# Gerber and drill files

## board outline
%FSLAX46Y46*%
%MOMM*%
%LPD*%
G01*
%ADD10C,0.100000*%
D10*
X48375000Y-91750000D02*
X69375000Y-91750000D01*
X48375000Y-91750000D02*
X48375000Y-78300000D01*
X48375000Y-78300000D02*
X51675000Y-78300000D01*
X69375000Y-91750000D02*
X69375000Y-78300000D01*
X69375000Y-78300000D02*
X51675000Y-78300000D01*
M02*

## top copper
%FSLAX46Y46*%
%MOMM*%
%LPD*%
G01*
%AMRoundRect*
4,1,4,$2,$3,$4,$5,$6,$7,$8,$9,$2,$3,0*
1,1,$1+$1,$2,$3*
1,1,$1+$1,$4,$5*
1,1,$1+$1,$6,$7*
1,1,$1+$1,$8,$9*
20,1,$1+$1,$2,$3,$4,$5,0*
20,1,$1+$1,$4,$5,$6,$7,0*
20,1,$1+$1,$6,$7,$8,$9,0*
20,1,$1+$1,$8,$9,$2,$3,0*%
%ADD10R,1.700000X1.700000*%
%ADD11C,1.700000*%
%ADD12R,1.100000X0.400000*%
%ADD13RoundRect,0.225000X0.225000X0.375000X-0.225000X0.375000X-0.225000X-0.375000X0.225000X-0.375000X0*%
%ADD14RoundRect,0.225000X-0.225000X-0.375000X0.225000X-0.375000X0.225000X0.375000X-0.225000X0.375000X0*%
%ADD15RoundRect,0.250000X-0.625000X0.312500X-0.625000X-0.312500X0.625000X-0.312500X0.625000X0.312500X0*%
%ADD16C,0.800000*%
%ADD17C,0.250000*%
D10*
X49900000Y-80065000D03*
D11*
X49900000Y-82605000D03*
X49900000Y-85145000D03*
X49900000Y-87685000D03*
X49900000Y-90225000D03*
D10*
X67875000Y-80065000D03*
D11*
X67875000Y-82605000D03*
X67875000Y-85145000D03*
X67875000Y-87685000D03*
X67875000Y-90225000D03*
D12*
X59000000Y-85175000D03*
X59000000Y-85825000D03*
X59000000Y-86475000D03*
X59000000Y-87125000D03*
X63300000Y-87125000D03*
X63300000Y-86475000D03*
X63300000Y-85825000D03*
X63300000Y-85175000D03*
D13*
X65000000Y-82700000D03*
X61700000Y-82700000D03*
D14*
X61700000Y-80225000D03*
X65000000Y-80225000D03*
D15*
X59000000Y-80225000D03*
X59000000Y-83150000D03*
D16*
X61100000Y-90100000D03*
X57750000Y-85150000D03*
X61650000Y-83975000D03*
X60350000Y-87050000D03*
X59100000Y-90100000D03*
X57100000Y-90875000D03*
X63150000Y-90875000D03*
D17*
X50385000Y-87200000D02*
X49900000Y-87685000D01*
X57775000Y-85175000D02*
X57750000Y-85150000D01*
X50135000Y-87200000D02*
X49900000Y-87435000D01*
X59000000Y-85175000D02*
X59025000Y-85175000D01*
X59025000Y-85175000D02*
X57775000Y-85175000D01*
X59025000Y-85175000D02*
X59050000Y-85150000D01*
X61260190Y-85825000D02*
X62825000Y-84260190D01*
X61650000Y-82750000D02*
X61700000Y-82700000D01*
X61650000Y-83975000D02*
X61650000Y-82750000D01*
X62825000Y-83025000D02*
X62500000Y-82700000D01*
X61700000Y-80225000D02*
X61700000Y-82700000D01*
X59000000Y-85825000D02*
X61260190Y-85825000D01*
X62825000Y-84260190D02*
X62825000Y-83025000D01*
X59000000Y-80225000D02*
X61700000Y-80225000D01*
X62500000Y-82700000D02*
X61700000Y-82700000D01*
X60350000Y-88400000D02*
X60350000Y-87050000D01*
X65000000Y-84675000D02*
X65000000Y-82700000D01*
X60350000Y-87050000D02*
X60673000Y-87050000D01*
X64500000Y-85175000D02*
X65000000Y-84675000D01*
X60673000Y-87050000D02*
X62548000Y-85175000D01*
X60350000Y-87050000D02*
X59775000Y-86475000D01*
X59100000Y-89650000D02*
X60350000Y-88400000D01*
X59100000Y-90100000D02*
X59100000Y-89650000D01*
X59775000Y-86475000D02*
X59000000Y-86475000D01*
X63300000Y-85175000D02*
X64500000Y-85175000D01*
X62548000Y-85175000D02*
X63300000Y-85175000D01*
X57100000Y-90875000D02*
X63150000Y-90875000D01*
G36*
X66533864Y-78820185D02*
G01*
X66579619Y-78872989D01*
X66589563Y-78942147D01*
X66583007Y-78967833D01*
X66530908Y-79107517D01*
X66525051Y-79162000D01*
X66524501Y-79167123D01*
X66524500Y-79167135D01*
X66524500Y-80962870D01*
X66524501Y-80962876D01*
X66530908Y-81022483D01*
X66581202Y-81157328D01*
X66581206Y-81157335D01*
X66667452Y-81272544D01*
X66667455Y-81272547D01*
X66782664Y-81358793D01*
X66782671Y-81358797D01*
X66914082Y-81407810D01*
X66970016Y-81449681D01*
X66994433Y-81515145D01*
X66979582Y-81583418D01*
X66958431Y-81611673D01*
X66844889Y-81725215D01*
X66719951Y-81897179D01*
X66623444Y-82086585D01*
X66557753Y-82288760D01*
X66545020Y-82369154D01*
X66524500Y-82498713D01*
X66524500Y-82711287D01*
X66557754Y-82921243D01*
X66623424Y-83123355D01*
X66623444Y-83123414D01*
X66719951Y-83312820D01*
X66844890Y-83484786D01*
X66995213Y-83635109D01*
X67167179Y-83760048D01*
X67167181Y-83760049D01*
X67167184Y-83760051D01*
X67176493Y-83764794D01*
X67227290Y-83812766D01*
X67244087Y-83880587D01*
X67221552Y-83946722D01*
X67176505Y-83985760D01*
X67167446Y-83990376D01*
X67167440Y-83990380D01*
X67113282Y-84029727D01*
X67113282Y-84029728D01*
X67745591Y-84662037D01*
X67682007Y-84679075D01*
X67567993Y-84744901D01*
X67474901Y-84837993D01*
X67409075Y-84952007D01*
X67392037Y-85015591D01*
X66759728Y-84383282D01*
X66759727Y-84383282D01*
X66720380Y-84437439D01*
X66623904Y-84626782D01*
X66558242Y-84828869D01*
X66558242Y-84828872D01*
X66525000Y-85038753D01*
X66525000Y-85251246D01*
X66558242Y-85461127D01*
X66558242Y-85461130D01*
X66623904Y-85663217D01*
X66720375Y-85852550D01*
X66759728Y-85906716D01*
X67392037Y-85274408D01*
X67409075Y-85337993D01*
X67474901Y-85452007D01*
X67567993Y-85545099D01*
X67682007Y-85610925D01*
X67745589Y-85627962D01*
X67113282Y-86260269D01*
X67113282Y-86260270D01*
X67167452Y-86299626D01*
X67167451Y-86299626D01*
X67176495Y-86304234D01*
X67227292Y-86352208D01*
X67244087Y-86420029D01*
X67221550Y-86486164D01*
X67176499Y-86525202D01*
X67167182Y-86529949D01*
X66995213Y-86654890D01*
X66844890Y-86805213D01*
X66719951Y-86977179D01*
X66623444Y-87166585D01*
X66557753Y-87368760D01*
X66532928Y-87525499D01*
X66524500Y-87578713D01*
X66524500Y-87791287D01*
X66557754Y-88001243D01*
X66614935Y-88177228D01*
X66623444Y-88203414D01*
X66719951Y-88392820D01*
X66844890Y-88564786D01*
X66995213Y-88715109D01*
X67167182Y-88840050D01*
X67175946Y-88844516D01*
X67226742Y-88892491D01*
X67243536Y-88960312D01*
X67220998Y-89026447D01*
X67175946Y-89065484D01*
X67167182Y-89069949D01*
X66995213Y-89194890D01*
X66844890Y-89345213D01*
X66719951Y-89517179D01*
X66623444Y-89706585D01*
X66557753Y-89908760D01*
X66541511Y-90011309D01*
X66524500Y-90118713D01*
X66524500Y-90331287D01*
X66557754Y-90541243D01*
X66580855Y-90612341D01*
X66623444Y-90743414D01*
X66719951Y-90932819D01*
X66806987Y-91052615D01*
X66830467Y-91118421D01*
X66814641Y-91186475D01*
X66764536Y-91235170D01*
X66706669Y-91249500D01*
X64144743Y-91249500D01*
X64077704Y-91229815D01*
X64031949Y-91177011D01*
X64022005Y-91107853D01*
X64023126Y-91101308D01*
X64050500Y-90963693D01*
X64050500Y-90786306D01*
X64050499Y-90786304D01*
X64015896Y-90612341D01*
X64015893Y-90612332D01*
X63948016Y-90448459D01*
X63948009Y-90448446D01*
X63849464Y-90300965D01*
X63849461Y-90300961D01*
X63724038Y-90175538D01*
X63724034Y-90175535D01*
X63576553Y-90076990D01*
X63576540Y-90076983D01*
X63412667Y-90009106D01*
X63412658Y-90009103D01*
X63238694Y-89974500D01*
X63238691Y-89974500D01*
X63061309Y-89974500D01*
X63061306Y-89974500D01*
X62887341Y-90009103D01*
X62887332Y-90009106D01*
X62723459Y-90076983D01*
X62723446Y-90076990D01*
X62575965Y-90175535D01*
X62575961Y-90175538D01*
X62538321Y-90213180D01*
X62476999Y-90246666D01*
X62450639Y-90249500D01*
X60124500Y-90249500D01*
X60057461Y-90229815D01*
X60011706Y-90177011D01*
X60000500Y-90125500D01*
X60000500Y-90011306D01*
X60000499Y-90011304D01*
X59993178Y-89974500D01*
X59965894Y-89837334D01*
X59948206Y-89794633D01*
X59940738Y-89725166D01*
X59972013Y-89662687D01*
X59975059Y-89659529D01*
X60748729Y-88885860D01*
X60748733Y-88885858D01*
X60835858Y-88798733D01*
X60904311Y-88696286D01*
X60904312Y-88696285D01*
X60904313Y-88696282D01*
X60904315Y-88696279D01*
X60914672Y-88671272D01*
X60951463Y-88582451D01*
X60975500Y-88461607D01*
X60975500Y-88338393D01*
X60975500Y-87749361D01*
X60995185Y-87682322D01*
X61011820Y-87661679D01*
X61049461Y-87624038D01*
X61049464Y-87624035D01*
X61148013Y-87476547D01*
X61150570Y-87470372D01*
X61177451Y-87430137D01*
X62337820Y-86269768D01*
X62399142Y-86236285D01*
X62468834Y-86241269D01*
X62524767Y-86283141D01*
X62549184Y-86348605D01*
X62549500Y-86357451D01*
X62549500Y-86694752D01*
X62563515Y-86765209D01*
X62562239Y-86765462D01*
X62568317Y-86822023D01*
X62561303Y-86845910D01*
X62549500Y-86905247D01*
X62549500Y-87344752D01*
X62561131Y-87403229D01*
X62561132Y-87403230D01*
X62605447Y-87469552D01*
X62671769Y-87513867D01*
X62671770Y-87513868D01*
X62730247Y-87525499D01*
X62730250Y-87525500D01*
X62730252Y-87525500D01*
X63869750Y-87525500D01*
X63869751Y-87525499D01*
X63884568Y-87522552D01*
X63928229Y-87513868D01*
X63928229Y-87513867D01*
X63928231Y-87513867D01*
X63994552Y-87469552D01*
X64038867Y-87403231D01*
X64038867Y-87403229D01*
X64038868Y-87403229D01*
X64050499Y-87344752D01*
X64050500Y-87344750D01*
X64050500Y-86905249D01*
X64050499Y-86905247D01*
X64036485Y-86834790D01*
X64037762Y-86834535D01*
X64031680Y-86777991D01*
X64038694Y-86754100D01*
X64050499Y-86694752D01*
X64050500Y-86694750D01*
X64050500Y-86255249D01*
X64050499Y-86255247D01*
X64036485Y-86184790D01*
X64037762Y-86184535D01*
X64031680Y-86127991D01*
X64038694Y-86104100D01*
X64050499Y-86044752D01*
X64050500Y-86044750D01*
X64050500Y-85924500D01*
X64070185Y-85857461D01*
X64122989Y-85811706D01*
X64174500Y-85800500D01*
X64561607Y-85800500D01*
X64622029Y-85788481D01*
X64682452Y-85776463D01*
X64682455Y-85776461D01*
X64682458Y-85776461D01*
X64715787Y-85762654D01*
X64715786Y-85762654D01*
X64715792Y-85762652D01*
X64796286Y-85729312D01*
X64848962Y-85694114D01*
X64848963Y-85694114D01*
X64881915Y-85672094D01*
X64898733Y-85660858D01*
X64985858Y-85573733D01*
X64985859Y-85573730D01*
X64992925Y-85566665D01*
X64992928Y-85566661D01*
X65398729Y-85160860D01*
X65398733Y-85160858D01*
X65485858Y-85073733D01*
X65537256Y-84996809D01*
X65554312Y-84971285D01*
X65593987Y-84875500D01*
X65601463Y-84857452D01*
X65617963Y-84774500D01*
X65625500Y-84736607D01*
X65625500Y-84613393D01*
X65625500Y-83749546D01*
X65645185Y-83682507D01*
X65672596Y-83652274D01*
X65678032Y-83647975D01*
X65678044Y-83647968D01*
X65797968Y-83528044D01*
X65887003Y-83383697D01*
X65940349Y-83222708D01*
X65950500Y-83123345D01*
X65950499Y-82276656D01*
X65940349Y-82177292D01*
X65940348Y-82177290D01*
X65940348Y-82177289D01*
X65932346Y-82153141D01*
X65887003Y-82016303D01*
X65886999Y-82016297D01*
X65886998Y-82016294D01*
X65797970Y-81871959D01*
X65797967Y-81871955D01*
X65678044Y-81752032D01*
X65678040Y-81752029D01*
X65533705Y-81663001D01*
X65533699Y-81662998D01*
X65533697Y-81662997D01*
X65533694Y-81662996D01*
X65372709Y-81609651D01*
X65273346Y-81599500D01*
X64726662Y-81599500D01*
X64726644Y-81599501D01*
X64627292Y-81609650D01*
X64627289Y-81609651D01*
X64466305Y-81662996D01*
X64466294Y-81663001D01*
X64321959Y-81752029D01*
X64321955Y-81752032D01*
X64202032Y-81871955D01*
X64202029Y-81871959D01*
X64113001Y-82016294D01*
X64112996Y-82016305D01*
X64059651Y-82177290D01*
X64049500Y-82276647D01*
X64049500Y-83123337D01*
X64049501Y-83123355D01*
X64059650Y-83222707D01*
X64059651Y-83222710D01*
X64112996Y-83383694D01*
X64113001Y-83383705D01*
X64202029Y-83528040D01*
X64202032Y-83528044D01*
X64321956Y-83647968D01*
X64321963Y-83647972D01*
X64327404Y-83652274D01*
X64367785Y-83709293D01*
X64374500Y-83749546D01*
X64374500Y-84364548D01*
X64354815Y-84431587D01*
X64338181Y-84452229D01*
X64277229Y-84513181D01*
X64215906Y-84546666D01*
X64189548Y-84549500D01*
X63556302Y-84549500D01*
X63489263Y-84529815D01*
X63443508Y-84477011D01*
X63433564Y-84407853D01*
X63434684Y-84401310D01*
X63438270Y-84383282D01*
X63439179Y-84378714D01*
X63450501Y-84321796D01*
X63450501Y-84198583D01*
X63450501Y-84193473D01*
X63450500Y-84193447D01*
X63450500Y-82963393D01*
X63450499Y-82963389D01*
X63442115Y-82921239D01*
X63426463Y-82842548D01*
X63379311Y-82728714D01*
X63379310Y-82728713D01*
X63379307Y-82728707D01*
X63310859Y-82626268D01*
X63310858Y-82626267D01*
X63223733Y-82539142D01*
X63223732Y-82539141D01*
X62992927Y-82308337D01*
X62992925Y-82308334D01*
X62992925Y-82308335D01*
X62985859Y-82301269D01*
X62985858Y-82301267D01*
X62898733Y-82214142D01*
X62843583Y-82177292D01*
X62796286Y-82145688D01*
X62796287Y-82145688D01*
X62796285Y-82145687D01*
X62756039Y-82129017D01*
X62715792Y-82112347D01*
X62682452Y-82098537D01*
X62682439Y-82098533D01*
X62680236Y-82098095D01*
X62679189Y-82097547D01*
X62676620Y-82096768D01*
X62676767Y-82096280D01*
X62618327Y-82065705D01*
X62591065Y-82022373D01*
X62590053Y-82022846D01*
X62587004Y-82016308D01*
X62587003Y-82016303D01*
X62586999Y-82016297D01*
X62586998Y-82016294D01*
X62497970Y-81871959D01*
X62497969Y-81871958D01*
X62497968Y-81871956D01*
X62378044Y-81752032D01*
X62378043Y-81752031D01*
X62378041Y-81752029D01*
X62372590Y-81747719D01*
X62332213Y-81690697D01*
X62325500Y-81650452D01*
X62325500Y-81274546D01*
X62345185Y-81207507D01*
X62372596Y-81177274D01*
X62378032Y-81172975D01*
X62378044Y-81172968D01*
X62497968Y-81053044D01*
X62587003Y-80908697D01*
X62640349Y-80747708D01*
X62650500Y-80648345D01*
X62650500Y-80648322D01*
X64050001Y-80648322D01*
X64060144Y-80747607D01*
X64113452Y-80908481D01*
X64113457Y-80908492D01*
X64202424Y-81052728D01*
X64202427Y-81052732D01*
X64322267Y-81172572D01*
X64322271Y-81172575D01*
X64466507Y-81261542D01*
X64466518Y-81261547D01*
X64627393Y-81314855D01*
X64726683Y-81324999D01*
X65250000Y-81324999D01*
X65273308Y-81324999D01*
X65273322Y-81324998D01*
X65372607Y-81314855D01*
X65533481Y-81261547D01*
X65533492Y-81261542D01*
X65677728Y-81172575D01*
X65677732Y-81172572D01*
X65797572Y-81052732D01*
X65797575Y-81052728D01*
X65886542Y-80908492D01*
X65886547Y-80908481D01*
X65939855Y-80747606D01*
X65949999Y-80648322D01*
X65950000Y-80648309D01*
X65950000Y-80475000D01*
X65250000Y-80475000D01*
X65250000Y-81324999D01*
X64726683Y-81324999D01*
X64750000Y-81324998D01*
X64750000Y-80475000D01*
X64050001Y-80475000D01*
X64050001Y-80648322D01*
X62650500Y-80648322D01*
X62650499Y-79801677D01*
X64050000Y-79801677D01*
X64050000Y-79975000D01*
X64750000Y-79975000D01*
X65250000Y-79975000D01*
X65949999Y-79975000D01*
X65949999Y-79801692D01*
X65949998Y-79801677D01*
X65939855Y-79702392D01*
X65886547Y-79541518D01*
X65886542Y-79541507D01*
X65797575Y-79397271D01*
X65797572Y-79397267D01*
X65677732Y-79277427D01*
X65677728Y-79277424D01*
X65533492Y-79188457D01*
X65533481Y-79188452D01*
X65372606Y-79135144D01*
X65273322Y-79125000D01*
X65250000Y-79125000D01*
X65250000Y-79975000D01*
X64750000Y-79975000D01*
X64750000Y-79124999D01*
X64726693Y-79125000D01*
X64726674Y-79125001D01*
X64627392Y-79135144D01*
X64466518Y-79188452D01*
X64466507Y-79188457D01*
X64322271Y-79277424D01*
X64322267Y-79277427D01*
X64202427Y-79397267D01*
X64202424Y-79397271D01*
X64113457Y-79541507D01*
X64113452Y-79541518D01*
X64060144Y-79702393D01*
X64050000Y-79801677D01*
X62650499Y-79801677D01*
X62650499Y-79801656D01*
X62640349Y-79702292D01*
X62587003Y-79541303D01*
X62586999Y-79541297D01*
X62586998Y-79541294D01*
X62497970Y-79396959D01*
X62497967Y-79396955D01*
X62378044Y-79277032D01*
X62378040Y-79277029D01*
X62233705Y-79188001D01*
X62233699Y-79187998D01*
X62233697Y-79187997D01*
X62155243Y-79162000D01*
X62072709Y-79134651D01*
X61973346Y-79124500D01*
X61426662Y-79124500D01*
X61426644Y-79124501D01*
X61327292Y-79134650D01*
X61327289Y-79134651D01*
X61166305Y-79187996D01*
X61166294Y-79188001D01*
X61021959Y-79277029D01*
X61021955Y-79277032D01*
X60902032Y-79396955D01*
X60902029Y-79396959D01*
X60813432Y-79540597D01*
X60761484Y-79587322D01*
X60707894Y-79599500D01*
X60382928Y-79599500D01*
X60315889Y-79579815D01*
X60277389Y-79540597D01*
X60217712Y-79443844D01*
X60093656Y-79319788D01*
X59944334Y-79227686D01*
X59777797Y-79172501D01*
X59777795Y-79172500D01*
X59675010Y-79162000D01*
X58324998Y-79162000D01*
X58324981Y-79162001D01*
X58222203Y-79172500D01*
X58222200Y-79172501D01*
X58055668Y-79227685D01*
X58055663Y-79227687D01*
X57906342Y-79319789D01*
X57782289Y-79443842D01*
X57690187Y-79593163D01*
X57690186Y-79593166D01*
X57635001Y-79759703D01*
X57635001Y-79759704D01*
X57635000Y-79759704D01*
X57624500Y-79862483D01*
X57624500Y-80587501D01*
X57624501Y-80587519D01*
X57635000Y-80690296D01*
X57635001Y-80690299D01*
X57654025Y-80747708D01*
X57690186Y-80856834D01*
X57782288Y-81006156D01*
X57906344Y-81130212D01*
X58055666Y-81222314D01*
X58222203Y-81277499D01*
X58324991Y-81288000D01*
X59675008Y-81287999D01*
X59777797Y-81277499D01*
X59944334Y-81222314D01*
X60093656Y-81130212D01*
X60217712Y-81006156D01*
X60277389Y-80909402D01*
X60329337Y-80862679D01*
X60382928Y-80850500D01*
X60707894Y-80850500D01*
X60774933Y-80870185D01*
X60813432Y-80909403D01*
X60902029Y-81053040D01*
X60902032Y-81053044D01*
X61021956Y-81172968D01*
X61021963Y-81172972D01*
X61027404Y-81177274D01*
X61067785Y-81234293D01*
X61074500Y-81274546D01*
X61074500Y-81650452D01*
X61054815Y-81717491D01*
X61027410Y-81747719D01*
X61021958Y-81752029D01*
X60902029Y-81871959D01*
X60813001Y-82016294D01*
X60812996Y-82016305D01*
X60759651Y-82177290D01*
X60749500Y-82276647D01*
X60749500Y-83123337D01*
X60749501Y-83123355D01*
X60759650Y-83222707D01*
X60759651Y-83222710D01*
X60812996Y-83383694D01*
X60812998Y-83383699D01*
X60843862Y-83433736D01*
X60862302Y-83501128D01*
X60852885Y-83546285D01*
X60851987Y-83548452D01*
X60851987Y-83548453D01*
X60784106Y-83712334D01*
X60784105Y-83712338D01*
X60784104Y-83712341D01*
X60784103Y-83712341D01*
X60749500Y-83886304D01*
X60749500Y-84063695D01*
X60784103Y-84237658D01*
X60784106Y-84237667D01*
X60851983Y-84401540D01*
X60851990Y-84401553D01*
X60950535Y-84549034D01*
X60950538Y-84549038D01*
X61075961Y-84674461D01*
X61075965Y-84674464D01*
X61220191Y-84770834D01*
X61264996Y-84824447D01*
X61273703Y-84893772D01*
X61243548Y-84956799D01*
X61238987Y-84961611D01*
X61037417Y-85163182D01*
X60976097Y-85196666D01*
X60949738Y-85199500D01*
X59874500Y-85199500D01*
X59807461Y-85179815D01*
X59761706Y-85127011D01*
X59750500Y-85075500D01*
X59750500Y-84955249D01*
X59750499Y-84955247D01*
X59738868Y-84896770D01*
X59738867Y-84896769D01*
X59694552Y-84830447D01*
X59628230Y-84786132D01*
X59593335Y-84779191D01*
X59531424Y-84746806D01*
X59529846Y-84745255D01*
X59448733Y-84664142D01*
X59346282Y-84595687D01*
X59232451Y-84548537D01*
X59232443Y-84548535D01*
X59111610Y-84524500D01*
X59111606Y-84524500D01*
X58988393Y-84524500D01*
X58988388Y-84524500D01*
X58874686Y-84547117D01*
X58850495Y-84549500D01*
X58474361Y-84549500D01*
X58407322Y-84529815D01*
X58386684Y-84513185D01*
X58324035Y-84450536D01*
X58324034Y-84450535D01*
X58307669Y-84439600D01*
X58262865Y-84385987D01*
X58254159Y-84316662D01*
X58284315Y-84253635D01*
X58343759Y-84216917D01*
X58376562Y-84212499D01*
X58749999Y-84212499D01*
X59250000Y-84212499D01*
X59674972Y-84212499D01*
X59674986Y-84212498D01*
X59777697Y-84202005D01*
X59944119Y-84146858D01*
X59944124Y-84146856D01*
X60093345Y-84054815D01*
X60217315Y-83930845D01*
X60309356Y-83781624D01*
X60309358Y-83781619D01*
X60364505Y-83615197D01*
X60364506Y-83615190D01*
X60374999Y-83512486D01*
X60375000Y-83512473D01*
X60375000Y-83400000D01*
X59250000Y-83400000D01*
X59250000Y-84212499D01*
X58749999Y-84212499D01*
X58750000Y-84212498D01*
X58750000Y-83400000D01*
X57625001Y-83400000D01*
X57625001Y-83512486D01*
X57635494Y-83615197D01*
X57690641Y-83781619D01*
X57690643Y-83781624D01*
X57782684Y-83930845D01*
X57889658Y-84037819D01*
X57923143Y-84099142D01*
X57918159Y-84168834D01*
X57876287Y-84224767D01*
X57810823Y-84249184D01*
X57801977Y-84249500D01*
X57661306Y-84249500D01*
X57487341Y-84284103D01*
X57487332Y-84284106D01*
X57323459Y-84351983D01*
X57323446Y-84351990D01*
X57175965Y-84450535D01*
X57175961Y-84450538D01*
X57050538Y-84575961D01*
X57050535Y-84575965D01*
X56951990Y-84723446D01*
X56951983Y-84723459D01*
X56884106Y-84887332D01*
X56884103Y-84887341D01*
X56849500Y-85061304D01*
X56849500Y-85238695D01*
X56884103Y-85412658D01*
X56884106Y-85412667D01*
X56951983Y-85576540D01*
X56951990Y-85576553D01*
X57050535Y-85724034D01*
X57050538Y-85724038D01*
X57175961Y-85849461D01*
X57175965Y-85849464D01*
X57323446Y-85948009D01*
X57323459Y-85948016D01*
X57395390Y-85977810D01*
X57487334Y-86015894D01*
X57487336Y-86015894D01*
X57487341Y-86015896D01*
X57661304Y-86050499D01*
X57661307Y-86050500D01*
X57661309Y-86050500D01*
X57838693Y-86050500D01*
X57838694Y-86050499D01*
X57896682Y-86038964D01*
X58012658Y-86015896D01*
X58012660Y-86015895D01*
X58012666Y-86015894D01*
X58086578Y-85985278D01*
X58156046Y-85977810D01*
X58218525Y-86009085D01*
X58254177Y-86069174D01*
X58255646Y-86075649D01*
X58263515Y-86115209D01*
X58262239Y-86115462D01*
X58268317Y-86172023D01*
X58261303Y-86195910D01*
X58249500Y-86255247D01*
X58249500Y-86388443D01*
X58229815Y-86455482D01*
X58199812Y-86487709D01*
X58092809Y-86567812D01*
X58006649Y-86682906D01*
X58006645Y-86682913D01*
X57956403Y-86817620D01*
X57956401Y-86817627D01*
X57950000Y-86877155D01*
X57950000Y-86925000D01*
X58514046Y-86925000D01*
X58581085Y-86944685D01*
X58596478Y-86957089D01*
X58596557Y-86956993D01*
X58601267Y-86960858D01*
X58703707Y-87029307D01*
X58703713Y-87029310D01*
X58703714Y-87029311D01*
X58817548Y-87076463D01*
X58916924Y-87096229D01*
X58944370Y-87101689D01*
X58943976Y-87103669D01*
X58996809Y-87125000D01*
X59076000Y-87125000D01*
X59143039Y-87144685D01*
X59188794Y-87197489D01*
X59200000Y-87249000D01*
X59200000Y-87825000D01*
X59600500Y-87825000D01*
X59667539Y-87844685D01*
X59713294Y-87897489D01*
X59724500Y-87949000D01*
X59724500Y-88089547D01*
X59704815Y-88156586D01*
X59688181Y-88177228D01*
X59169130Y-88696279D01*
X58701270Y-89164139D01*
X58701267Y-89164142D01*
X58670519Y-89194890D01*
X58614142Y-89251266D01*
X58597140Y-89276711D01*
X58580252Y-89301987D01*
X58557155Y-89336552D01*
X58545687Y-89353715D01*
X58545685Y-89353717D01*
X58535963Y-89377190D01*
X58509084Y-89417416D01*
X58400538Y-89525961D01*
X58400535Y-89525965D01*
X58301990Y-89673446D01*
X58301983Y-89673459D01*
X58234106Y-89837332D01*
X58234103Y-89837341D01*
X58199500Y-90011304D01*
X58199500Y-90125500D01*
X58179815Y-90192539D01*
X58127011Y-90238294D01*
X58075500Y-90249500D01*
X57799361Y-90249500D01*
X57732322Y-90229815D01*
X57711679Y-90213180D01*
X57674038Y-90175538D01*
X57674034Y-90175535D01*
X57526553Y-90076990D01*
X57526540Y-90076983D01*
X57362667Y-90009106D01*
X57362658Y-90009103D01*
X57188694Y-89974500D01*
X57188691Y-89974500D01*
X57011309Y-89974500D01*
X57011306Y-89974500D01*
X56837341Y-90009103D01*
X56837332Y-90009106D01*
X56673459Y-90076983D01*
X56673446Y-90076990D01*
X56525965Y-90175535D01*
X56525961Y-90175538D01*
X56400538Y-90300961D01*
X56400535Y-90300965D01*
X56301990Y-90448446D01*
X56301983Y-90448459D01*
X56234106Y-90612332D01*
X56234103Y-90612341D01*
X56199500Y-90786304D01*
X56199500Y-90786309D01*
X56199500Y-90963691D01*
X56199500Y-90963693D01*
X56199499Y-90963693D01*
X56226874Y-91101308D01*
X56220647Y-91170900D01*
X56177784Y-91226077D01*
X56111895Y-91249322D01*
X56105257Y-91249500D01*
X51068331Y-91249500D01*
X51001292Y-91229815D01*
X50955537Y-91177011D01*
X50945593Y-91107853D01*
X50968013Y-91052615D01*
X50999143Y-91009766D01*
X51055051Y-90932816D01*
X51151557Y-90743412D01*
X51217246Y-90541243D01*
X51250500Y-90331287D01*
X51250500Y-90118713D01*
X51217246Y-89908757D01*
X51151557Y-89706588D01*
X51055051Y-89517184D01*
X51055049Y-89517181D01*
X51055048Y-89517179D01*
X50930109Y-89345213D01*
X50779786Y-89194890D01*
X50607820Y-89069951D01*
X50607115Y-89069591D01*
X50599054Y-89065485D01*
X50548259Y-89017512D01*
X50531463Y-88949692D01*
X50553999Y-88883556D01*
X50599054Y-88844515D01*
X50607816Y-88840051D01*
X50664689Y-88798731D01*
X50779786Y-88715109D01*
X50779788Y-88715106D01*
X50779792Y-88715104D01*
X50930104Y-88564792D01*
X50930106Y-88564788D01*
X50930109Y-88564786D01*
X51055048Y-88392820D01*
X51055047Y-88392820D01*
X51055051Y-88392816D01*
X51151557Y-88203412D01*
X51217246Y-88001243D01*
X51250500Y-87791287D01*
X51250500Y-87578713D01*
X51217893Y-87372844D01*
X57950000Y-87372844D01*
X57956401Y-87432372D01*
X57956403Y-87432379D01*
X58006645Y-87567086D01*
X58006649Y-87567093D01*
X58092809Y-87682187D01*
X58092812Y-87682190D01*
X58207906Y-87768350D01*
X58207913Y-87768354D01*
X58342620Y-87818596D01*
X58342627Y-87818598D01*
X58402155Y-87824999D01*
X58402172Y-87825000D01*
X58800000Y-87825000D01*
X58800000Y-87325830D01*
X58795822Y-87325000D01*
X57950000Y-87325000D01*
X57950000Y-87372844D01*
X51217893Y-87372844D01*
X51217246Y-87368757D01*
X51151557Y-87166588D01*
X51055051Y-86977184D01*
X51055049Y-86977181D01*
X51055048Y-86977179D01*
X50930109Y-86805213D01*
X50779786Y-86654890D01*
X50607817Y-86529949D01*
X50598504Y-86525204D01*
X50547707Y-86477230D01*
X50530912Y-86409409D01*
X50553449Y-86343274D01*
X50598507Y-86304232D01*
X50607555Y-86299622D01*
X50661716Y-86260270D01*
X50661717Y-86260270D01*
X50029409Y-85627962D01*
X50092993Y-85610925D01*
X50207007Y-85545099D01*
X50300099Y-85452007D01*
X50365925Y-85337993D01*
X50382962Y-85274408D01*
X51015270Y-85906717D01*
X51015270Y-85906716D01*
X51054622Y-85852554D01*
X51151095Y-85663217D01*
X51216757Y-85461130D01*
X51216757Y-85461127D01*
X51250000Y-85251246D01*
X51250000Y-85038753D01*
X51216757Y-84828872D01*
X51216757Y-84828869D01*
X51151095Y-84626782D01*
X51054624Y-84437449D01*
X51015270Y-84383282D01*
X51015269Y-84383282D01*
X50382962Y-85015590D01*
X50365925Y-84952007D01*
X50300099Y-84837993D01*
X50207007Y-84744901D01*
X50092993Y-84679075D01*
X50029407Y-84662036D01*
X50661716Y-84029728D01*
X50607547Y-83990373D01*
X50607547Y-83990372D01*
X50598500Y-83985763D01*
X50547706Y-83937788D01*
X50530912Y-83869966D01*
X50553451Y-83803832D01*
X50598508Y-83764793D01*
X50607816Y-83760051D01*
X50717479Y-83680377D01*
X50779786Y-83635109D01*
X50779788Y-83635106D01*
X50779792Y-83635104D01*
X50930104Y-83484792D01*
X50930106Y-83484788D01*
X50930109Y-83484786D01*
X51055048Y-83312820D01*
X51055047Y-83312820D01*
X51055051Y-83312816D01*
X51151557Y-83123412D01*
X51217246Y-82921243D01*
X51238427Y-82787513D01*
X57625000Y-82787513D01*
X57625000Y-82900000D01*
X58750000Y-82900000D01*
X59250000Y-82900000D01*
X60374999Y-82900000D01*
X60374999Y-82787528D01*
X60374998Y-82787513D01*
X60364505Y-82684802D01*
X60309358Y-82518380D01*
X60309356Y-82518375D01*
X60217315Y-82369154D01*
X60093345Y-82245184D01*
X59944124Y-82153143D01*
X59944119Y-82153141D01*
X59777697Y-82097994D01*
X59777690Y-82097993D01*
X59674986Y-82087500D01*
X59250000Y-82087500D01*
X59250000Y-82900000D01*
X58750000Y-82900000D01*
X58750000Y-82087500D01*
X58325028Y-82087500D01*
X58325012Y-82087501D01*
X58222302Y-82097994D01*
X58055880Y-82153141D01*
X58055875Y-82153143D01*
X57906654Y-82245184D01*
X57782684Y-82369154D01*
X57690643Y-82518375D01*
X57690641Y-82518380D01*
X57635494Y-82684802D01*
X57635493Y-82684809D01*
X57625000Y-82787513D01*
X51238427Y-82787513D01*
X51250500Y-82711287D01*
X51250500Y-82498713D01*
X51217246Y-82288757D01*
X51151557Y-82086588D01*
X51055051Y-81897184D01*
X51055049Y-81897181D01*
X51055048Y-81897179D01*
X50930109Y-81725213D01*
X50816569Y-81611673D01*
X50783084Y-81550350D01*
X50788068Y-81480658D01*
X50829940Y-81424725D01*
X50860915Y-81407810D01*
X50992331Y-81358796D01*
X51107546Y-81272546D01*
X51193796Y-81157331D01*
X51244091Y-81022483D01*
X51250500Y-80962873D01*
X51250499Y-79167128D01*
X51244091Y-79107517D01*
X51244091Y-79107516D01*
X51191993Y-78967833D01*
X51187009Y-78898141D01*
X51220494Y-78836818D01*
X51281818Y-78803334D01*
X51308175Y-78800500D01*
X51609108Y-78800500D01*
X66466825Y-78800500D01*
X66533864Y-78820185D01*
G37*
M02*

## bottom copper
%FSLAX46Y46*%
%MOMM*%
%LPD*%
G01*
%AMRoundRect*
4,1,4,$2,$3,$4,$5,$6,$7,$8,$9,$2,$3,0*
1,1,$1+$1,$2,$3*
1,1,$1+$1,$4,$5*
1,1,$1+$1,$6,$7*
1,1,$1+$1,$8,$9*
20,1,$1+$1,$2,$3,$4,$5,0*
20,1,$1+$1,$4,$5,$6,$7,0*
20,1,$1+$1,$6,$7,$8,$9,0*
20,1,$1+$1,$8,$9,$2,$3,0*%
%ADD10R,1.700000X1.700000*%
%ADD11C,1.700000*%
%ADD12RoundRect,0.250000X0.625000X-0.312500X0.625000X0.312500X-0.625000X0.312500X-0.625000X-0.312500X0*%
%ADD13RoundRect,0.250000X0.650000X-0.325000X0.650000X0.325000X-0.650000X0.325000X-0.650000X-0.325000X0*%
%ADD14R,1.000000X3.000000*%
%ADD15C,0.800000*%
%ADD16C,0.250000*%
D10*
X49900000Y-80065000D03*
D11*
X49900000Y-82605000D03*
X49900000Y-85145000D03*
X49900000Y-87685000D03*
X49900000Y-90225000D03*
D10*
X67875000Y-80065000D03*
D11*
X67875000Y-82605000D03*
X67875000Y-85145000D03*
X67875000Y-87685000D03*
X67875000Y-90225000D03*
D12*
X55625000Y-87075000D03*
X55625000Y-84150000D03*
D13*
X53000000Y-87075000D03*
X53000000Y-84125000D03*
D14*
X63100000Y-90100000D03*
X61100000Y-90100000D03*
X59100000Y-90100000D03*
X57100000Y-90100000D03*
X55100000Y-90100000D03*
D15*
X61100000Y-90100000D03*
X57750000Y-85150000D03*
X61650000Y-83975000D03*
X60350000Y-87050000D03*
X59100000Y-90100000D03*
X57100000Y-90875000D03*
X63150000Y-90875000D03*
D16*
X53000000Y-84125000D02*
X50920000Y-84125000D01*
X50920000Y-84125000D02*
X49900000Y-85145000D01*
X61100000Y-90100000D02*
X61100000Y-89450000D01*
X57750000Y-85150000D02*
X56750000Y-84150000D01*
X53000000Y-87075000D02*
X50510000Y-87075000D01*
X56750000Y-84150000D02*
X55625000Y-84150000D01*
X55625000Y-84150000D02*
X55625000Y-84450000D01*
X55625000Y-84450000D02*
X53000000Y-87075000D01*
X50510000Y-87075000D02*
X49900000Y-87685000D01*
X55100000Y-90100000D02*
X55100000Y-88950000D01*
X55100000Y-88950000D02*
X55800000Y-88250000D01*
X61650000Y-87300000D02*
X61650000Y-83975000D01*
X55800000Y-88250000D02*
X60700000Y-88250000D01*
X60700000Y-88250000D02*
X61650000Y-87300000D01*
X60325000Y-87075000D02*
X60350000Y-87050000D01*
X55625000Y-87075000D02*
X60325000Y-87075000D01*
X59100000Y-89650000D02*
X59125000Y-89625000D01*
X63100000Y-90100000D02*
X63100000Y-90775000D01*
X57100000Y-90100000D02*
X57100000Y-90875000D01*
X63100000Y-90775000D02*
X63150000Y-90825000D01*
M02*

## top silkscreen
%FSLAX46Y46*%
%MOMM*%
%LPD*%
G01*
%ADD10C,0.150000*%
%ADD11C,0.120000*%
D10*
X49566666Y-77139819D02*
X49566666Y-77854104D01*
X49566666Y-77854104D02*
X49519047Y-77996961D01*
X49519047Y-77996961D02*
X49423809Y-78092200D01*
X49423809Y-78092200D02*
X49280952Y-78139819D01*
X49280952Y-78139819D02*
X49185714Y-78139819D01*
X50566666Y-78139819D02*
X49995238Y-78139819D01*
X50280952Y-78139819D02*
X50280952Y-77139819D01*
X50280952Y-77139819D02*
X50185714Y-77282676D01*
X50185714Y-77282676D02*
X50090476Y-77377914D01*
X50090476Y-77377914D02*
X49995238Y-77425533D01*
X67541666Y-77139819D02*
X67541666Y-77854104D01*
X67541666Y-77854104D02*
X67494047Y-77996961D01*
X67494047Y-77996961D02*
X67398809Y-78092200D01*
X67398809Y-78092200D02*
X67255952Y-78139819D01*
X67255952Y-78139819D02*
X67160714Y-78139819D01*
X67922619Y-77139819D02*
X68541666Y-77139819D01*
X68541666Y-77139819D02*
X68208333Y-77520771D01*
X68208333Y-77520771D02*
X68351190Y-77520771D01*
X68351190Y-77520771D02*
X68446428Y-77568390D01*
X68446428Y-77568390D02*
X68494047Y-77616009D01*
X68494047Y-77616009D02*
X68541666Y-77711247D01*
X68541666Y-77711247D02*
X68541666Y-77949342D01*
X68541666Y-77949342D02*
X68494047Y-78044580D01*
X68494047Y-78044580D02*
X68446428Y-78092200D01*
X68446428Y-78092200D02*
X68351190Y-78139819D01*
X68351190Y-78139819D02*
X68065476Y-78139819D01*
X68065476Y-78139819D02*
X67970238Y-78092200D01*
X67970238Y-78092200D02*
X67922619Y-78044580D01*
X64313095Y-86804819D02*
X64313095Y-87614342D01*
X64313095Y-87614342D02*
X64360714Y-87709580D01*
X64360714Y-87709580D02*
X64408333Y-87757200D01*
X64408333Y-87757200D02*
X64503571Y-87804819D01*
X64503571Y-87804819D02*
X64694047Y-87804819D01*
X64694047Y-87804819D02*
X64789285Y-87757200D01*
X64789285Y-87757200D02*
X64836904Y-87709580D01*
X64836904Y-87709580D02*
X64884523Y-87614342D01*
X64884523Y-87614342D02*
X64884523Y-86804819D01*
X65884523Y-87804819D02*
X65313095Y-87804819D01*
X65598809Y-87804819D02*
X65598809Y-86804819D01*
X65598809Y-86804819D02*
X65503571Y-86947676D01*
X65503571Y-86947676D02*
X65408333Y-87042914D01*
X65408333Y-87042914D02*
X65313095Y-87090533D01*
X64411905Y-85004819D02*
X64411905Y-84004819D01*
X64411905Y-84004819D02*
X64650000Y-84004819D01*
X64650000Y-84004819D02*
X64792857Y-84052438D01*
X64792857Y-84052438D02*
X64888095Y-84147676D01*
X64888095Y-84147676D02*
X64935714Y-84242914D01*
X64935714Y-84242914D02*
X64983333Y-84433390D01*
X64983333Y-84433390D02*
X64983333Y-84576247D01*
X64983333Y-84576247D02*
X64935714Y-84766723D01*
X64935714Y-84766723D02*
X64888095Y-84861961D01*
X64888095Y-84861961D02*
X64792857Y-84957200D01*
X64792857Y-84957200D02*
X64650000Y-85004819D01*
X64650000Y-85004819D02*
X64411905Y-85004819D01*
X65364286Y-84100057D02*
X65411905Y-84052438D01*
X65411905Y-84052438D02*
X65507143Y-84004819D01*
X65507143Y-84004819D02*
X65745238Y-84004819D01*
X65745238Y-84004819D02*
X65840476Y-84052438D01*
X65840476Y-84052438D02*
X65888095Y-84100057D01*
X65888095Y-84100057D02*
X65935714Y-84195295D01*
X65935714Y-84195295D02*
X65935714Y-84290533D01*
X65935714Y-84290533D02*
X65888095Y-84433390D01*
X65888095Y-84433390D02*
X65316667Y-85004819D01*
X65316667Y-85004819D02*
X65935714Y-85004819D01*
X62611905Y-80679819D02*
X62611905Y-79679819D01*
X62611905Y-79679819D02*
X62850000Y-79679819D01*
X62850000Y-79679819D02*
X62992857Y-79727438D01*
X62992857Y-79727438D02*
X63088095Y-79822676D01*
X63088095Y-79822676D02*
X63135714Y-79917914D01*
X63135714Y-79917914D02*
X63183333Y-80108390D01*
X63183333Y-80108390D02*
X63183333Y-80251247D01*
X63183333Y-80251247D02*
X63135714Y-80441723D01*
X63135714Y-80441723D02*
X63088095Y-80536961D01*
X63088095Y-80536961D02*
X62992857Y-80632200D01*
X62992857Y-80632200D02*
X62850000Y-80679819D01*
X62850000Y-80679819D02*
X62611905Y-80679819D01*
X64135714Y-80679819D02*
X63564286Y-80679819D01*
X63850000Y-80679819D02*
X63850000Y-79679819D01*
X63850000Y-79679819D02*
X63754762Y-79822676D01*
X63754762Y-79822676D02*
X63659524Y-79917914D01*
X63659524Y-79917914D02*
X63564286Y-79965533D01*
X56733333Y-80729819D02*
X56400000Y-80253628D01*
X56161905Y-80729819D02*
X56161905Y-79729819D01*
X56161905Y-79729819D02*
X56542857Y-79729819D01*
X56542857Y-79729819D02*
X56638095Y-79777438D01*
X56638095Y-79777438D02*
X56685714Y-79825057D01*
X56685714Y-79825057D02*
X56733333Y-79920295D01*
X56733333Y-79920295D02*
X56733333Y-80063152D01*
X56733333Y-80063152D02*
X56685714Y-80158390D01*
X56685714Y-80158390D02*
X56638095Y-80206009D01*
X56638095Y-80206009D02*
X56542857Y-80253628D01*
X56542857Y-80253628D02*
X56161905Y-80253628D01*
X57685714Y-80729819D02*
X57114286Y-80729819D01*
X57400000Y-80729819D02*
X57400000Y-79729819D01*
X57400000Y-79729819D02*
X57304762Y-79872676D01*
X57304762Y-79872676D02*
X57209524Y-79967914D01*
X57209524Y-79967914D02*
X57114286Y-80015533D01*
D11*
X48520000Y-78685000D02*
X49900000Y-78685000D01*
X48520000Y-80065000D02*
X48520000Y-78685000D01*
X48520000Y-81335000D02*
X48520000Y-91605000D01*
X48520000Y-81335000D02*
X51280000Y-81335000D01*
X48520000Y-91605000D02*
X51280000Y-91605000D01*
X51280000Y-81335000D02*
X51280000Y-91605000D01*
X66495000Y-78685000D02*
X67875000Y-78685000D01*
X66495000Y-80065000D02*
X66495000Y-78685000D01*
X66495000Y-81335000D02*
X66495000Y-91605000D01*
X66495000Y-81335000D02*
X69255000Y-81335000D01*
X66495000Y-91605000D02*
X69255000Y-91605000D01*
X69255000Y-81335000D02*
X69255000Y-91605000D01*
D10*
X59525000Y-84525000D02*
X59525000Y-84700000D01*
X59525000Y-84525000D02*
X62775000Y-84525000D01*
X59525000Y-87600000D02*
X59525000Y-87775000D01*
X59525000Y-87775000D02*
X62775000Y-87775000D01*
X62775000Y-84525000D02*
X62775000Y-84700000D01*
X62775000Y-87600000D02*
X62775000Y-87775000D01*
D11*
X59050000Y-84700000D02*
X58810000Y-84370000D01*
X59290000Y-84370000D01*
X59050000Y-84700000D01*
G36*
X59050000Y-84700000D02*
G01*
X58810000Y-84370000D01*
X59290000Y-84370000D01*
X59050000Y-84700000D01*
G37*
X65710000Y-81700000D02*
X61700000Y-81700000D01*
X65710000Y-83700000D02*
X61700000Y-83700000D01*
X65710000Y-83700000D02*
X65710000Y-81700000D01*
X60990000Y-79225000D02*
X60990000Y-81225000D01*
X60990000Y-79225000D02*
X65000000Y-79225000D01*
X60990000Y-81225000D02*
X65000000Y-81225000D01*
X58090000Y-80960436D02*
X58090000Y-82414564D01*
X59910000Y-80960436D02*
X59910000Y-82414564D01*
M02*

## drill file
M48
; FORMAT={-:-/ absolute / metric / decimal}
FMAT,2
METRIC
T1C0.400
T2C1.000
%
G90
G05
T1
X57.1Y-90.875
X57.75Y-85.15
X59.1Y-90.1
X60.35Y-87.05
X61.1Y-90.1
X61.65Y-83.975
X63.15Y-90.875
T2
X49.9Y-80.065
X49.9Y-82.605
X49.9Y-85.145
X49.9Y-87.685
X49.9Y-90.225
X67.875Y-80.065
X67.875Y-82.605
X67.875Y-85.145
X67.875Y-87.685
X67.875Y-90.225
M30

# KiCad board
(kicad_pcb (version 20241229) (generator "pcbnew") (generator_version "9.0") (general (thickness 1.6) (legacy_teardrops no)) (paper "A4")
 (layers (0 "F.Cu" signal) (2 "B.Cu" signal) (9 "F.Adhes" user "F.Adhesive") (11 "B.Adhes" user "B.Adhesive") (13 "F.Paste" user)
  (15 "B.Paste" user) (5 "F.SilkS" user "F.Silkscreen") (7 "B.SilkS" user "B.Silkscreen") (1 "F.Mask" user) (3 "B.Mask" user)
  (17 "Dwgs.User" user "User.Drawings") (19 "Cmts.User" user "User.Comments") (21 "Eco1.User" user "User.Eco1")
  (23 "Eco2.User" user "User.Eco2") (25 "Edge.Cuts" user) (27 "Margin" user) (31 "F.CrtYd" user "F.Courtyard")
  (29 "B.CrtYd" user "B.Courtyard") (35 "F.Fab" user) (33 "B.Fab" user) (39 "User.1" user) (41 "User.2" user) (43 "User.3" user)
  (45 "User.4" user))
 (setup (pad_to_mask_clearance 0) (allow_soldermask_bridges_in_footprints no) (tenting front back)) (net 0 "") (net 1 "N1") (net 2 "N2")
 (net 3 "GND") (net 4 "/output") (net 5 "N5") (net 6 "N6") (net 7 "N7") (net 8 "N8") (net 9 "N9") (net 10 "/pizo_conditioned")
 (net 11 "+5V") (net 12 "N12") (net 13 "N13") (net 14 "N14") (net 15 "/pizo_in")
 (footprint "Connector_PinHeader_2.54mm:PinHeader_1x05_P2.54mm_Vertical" (layer "F.Cu") (at 49.9 80.065)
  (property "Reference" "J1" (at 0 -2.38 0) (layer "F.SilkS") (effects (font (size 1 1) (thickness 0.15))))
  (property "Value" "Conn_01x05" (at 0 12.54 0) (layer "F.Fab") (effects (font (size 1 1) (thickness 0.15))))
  (fp_line (start -1.38 -1.38) (end 0 -1.38) (stroke (width 0.12) (type solid)) (layer "F.SilkS"))
  (fp_line (start -1.38 0) (end -1.38 -1.38) (stroke (width 0.12) (type solid)) (layer "F.SilkS"))
  (fp_line (start -1.38 1.27) (end -1.38 11.54) (stroke (width 0.12) (type solid)) (layer "F.SilkS"))
  (fp_line (start -1.38 1.27) (end 1.38 1.27) (stroke (width 0.12) (type solid)) (layer "F.SilkS"))
  (fp_line (start -1.38 11.54) (end 1.38 11.54) (stroke (width 0.12) (type solid)) (layer "F.SilkS"))
  (fp_line (start 1.38 1.27) (end 1.38 11.54) (stroke (width 0.12) (type solid)) (layer "F.SilkS"))
  (pad "1" thru_hole rect (at 0 0) (size 1.7 1.7) (drill 1) (layers "*.Cu" "*.Mask") (remove_unused_layers no) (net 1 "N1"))
  (pad "2" thru_hole circle (at 0 2.54) (size 1.7 1.7) (drill 1) (layers "*.Cu" "*.Mask") (remove_unused_layers no) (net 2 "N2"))
  (pad "3" thru_hole circle (at 0 5.08) (size 1.7 1.7) (drill 1) (layers "*.Cu" "*.Mask") (remove_unused_layers no) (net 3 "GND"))
  (pad "4" thru_hole circle (at 0 7.62) (size 1.7 1.7) (drill 1) (layers "*.Cu" "*.Mask") (remove_unused_layers no) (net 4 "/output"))
  (pad "5" thru_hole circle (at 0 10.16) (size 1.7 1.7) (drill 1) (layers "*.Cu" "*.Mask") (remove_unused_layers no) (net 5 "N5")))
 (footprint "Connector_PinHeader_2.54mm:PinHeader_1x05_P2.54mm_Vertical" (layer "F.Cu") (at 67.875 80.065)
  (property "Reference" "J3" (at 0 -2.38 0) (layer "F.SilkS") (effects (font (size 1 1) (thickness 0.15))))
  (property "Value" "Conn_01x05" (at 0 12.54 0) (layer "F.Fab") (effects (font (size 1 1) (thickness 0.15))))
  (fp_line (start -1.38 -1.38) (end 0 -1.38) (stroke (width 0.12) (type solid)) (layer "F.SilkS"))
  (fp_line (start -1.38 0) (end -1.38 -1.38) (stroke (width 0.12) (type solid)) (layer "F.SilkS"))
  (fp_line (start -1.38 1.27) (end -1.38 11.54) (stroke (width 0.12) (type solid)) (layer "F.SilkS"))
  (fp_line (start -1.38 1.27) (end 1.38 1.27) (stroke (width 0.12) (type solid)) (layer "F.SilkS"))
  (fp_line (start -1.38 11.54) (end 1.38 11.54) (stroke (width 0.12) (type solid)) (layer "F.SilkS"))
  (fp_line (start 1.38 1.27) (end 1.38 11.54) (stroke (width 0.12) (type solid)) (layer "F.SilkS"))
  (pad "1" thru_hole rect (at 0 0) (size 1.7 1.7) (drill 1) (layers "*.Cu" "*.Mask") (remove_unused_layers no) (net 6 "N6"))
  (pad "2" thru_hole circle (at 0 2.54) (size 1.7 1.7) (drill 1) (layers "*.Cu" "*.Mask") (remove_unused_layers no) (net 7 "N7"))
  (pad "3" thru_hole circle (at 0 5.08) (size 1.7 1.7) (drill 1) (layers "*.Cu" "*.Mask") (remove_unused_layers no) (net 3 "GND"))
  (pad "4" thru_hole circle (at 0 7.62) (size 1.7 1.7) (drill 1) (layers "*.Cu" "*.Mask") (remove_unused_layers no) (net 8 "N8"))
  (pad "5" thru_hole circle (at 0 10.16) (size 1.7 1.7) (drill 1) (layers "*.Cu" "*.Mask") (remove_unused_layers no) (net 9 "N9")))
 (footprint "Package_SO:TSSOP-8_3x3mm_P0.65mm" (layer "F.Cu") (at 61.15 86.15)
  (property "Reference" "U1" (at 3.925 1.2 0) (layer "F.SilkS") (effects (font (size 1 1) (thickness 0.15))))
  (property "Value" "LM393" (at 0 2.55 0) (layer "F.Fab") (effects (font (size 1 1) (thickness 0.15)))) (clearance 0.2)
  (fp_line (start -1.625 -1.625) (end -1.625 -1.45) (stroke (width 0.15) (type solid)) (layer "F.SilkS"))
  (fp_line (start -1.625 -1.625) (end 1.625 -1.625) (stroke (width 0.15) (type solid)) (layer "F.SilkS"))
  (fp_line (start -1.625 1.45) (end -1.625 1.625) (stroke (width 0.15) (type solid)) (layer "F.SilkS"))
  (fp_line (start -1.625 1.625) (end 1.625 1.625) (stroke (width 0.15) (type solid)) (layer "F.SilkS"))
  (fp_line (start 1.625 -1.625) (end 1.625 -1.45) (stroke (width 0.15) (type solid)) (layer "F.SilkS"))
  (fp_line (start 1.625 1.45) (end 1.625 1.625) (stroke (width 0.15) (type solid)) (layer "F.SilkS"))
  (fp_poly
   (pts (xy -2.1 -1.45) (xy -2.34 -1.78) (xy -1.86 -1.78) (xy -2.1 -1.45)) (stroke (width 0.12) (type solid)) (fill yes) (layer "F.SilkS"))
  (pad "1" smd rect (at -2.15 -0.975) (size 1.1 0.4) (layers "F.Cu" "F.Mask" "F.Paste") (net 4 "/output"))
  (pad "2" smd rect (at -2.15 -0.325) (size 1.1 0.4) (layers "F.Cu" "F.Mask" "F.Paste") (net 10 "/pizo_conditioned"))
  (pad "3" smd rect (at -2.15 0.325) (size 1.1 0.4) (layers "F.Cu" "F.Mask" "F.Paste") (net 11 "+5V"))
  (pad "4" smd rect (at -2.15 0.975) (size 1.1 0.4) (layers "F.Cu" "F.Mask" "F.Paste") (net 3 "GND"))
  (pad "5" smd rect (at 2.15 0.975) (size 1.1 0.4) (layers "F.Cu" "F.Mask" "F.Paste") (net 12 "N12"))
  (pad "6" smd rect (at 2.15 0.325) (size 1.1 0.4) (layers "F.Cu" "F.Mask" "F.Paste") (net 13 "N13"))
  (pad "7" smd rect (at 2.15 -0.325) (size 1.1 0.4) (layers "F.Cu" "F.Mask" "F.Paste") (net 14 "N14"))
  (pad "8" smd rect (at 2.15 -0.975) (size 1.1 0.4) (layers "F.Cu" "F.Mask" "F.Paste") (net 11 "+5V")))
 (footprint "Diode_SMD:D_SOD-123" (layer "F.Cu") (at 63.35 82.7 180)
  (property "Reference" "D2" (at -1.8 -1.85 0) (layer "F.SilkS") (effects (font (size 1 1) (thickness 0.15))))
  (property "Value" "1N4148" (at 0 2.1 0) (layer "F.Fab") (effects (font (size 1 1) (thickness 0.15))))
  (fp_line (start -2.36 1) (end 1.65 1) (stroke (width 0.12) (type solid)) (layer "F.SilkS"))
  (fp_line (start -2.36 -1) (end 1.65 -1) (stroke (width 0.12) (type solid)) (layer "F.SilkS"))
  (fp_line (start -2.36 -1) (end -2.36 1) (stroke (width 0.12) (type solid)) (layer "F.SilkS"))
  (pad "1" smd roundrect (at -1.65 0 180) (size 0.9 1.2) (layers "F.Cu" "F.Mask" "F.Paste") (roundrect_rratio 0.25) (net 11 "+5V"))
  (pad "2" smd roundrect (at 1.65 0 180) (size 0.9 1.2) (layers "F.Cu" "F.Mask" "F.Paste") (roundrect_rratio 0.25)
   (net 10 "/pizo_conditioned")))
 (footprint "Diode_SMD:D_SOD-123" (layer "F.Cu") (at 63.35 80.225)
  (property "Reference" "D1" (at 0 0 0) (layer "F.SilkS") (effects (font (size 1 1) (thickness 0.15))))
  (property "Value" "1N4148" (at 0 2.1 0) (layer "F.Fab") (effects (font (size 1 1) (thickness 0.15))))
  (fp_line (start -2.36 -1) (end -2.36 1) (stroke (width 0.12) (type solid)) (layer "F.SilkS"))
  (fp_line (start -2.36 -1) (end 1.65 -1) (stroke (width 0.12) (type solid)) (layer "F.SilkS"))
  (fp_line (start -2.36 1) (end 1.65 1) (stroke (width 0.12) (type solid)) (layer "F.SilkS"))
  (pad "1" smd roundrect (at -1.65 0) (size 0.9 1.2) (layers "F.Cu" "F.Mask" "F.Paste") (roundrect_rratio 0.25) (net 10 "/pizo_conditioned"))
  (pad "2" smd roundrect (at 1.65 0) (size 0.9 1.2) (layers "F.Cu" "F.Mask" "F.Paste") (roundrect_rratio 0.25) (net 3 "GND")))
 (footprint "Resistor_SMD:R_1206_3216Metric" (layer "F.Cu") (at 59 81.6875 -90)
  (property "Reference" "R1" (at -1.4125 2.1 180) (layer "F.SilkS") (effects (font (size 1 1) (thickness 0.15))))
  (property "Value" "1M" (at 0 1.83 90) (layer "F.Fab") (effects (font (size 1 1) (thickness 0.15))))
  (fp_line (start -0.727064 0.91) (end 0.727064 0.91) (stroke (width 0.12) (type solid)) (layer "F.SilkS"))
  (fp_line (start -0.727064 -0.91) (end 0.727064 -0.91) (stroke (width 0.12) (type solid)) (layer "F.SilkS"))
  (pad "1" smd roundrect (at -1.4625 0 270) (size 1.125 1.75) (layers "F.Cu" "F.Mask" "F.Paste") (roundrect_rratio 0.222222)
   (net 10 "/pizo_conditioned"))
  (pad "2" smd roundrect (at 1.4625 0 270) (size 1.125 1.75) (layers "F.Cu" "F.Mask" "F.Paste") (roundrect_rratio 0.222222) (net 3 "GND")))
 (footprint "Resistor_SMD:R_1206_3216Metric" (layer "B.Cu") (at 55.625 85.6125 90)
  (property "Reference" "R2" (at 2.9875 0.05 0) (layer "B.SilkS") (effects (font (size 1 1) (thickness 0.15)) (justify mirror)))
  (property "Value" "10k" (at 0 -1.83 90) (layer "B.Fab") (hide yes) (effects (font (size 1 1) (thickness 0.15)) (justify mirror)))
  (pad "1" smd roundrect (at -1.4625 0 90) (size 1.125 1.75) (layers "B.Cu" "B.Mask" "B.Paste") (roundrect_rratio 0.222222) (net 11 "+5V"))
  (pad "2" smd roundrect (at 1.4625 0 90) (size 1.125 1.75) (layers "B.Cu" "B.Mask" "B.Paste") (roundrect_rratio 0.222222) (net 4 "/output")))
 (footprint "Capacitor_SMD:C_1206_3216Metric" (layer "B.Cu") (at 53 85.6 90)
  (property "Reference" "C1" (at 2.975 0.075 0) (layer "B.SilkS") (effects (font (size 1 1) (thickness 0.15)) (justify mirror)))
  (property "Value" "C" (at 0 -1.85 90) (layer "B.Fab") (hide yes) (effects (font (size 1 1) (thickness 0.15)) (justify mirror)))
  (pad "1" smd roundrect (at -1.475 0 90) (size 1.15 1.8) (layers "B.Cu" "B.Mask" "B.Paste") (roundrect_rratio 0.217391) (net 4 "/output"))
  (pad "2" smd roundrect (at 1.475 0 90) (size 1.15 1.8) (layers "B.Cu" "B.Mask" "B.Paste") (roundrect_rratio 0.217391) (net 3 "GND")))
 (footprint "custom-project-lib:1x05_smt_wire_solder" (layer "B.Cu") (at 63.1 90.1 180)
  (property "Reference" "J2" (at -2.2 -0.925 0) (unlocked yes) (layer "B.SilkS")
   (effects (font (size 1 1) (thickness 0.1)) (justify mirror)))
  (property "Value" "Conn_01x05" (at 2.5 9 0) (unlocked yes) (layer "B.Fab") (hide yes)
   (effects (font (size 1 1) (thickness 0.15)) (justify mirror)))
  (pad "1" smd rect (at 0 0 180) (size 1 3) (layers "B.Cu" "B.Mask" "B.Paste") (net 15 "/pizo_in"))
  (pad "2" smd rect (at 2 0 180) (size 1 3) (layers "B.Cu" "B.Mask" "B.Paste") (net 3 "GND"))
  (pad "3" smd rect (at 4 0 180) (size 1 3) (layers "B.Cu" "B.Mask" "B.Paste") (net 11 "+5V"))
  (pad "4" smd rect (at 6 0 180) (size 1 3) (layers "B.Cu" "B.Mask" "B.Paste") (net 15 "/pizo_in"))
  (pad "5" smd rect (at 8 0 180) (size 1 3) (layers "B.Cu" "B.Mask" "B.Paste") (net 10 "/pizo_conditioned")))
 (gr_line (start 48.375 91.75) (end 69.375 91.75) (stroke (width 0.1) (type default)) (layer "Edge.Cuts"))
 (gr_line (start 48.375 91.75) (end 48.375 78.3) (stroke (width 0.1) (type default)) (layer "Edge.Cuts"))
 (gr_line (start 48.375 78.3) (end 51.675 78.3) (stroke (width 0.1) (type default)) (layer "Edge.Cuts"))
 (gr_line (start 69.375 91.75) (end 69.375 78.3) (stroke (width 0.1) (type default)) (layer "Edge.Cuts"))
 (gr_line (start 69.375 78.3) (end 51.675 78.3) (stroke (width 0.1) (type default)) (layer "Edge.Cuts"))
 (via (at 61.1 90.1) (size 0.8) (drill 0.4) (layers "F.Cu" "B.Cu") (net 3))
 (segment (start 53 84.125) (end 50.92 84.125) (width 0.25) (layer "B.Cu") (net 3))
 (segment (start 50.92 84.125) (end 49.9 85.145) (width 0.25) (layer "B.Cu") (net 3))
 (segment (start 61.1 90.1) (end 61.1 89.45) (width 0.25) (layer "B.Cu") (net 3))
 (segment (start 50.385 87.2) (end 49.9 87.685) (width 0.25) (layer "F.Cu") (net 4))
 (segment (start 57.775 85.175) (end 57.75 85.15) (width 0.25) (layer "F.Cu") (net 4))
 (segment (start 50.135 87.2) (end 49.9 87.435) (width 0.25) (layer "F.Cu") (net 4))
 (segment (start 59 85.175) (end 59.025 85.175) (width 0.25) (layer "F.Cu") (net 4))
 (segment (start 59.025 85.175) (end 57.775 85.175) (width 0.25) (layer "F.Cu") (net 4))
 (segment (start 59.025 85.175) (end 59.05 85.15) (width 0.25) (layer "F.Cu") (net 4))
 (via (at 57.75 85.15) (size 0.8) (drill 0.4) (layers "F.Cu" "B.Cu") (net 4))
 (segment (start 57.75 85.15) (end 56.75 84.15) (width 0.25) (layer "B.Cu") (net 4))
 (segment (start 53 87.075) (end 50.51 87.075) (width 0.25) (layer "B.Cu") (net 4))
 (segment (start 56.75 84.15) (end 55.625 84.15) (width 0.25) (layer "B.Cu") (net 4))
 (segment (start 55.625 84.15) (end 55.625 84.45) (width 0.25) (layer "B.Cu") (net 4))
 (segment (start 55.625 84.45) (end 53 87.075) (width 0.25) (layer "B.Cu") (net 4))
 (segment (start 50.51 87.075) (end 49.9 87.685) (width 0.25) (layer "B.Cu") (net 4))
 (segment (start 61.26019 85.825) (end 62.825 84.26019) (width 0.25) (layer "F.Cu") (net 10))
 (segment (start 61.65 82.75) (end 61.7 82.7) (width 0.25) (layer "F.Cu") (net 10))
 (segment (start 61.65 83.975) (end 61.65 82.75) (width 0.25) (layer "F.Cu") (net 10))
 (segment (start 62.825 83.025) (end 62.5 82.7) (width 0.25) (layer "F.Cu") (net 10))
 (segment (start 61.7 80.225) (end 61.7 82.7) (width 0.25) (layer "F.Cu") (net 10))
 (segment (start 59 85.825) (end 61.26019 85.825) (width 0.25) (layer "F.Cu") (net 10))
 (segment (start 62.825 84.26019) (end 62.825 83.025) (width 0.25) (layer "F.Cu") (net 10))
 (segment (start 59 80.225) (end 61.7 80.225) (width 0.25) (layer "F.Cu") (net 10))
 (segment (start 62.5 82.7) (end 61.7 82.7) (width 0.25) (layer "F.Cu") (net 10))
 (via (at 61.65 83.975) (size 0.8) (drill 0.4) (layers "F.Cu" "B.Cu") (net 10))
 (segment (start 55.1 90.1) (end 55.1 88.95) (width 0.25) (layer "B.Cu") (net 10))
 (segment (start 55.1 88.95) (end 55.8 88.25) (width 0.25) (layer "B.Cu") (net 10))
 (segment (start 61.65 87.3) (end 61.65 83.975) (width 0.25) (layer "B.Cu") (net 10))
 (segment (start 55.8 88.25) (end 60.7 88.25) (width 0.25) (layer "B.Cu") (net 10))
 (segment (start 60.7 88.25) (end 61.65 87.3) (width 0.25) (layer "B.Cu") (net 10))
 (segment (start 60.35 88.4) (end 60.35 87.05) (width 0.25) (layer "F.Cu") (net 11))
 (segment (start 65 84.675) (end 65 82.7) (width 0.25) (layer "F.Cu") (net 11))
 (segment (start 60.35 87.05) (end 60.673 87.05) (width 0.25) (layer "F.Cu") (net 11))
 (segment (start 64.5 85.175) (end 65 84.675) (width 0.25) (layer "F.Cu") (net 11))
 (segment (start 60.673 87.05) (end 62.548 85.175) (width 0.25) (layer "F.Cu") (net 11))
 (segment (start 60.35 87.05) (end 59.775 86.475) (width 0.25) (layer "F.Cu") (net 11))
 (segment (start 59.1 89.65) (end 60.35 88.4) (width 0.25) (layer "F.Cu") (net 11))
 (segment (start 59.1 90.1) (end 59.1 89.65) (width 0.25) (layer "F.Cu") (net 11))
 (segment (start 59.775 86.475) (end 59 86.475) (width 0.25) (layer "F.Cu") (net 11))
 (segment (start 63.3 85.175) (end 64.5 85.175) (width 0.25) (layer "F.Cu") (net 11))
 (segment (start 62.548 85.175) (end 63.3 85.175) (width 0.25) (layer "F.Cu") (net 11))
 (via (at 60.35 87.05) (size 0.8) (drill 0.4) (layers "F.Cu" "B.Cu") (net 11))
 (via (at 59.1 90.1) (size 0.8) (drill 0.4) (layers "F.Cu" "B.Cu") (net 11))
 (segment (start 60.325 87.075) (end 60.35 87.05) (width 0.25) (layer "B.Cu") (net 11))
 (segment (start 55.625 87.075) (end 60.325 87.075) (width 0.25) (layer "B.Cu") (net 11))
 (segment (start 59.1 89.65) (end 59.125 89.625) (width 0.25) (layer "B.Cu") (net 11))
 (segment (start 57.1 90.875) (end 63.15 90.875) (width 0.25) (layer "F.Cu") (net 15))
 (via (at 57.1 90.875) (size 0.8) (drill 0.4) (layers "F.Cu" "B.Cu") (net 15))
 (via (at 63.15 90.875) (size 0.8) (drill 0.4) (layers "F.Cu" "B.Cu") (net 15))
 (segment (start 63.1 90.1) (end 63.1 90.775) (width 0.25) (layer "B.Cu") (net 15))
 (segment (start 57.1 90.1) (end 57.1 90.875) (width 0.25) (layer "B.Cu") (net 15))
 (segment (start 63.1 90.775) (end 63.15 90.825) (width 0.25) (layer "B.Cu") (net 15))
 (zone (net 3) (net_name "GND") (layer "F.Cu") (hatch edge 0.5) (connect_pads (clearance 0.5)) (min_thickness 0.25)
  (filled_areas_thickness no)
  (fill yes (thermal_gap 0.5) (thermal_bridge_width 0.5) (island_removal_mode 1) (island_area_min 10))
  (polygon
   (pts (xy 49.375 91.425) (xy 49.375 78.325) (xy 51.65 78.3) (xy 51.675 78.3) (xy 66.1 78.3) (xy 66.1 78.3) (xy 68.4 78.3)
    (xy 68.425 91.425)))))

